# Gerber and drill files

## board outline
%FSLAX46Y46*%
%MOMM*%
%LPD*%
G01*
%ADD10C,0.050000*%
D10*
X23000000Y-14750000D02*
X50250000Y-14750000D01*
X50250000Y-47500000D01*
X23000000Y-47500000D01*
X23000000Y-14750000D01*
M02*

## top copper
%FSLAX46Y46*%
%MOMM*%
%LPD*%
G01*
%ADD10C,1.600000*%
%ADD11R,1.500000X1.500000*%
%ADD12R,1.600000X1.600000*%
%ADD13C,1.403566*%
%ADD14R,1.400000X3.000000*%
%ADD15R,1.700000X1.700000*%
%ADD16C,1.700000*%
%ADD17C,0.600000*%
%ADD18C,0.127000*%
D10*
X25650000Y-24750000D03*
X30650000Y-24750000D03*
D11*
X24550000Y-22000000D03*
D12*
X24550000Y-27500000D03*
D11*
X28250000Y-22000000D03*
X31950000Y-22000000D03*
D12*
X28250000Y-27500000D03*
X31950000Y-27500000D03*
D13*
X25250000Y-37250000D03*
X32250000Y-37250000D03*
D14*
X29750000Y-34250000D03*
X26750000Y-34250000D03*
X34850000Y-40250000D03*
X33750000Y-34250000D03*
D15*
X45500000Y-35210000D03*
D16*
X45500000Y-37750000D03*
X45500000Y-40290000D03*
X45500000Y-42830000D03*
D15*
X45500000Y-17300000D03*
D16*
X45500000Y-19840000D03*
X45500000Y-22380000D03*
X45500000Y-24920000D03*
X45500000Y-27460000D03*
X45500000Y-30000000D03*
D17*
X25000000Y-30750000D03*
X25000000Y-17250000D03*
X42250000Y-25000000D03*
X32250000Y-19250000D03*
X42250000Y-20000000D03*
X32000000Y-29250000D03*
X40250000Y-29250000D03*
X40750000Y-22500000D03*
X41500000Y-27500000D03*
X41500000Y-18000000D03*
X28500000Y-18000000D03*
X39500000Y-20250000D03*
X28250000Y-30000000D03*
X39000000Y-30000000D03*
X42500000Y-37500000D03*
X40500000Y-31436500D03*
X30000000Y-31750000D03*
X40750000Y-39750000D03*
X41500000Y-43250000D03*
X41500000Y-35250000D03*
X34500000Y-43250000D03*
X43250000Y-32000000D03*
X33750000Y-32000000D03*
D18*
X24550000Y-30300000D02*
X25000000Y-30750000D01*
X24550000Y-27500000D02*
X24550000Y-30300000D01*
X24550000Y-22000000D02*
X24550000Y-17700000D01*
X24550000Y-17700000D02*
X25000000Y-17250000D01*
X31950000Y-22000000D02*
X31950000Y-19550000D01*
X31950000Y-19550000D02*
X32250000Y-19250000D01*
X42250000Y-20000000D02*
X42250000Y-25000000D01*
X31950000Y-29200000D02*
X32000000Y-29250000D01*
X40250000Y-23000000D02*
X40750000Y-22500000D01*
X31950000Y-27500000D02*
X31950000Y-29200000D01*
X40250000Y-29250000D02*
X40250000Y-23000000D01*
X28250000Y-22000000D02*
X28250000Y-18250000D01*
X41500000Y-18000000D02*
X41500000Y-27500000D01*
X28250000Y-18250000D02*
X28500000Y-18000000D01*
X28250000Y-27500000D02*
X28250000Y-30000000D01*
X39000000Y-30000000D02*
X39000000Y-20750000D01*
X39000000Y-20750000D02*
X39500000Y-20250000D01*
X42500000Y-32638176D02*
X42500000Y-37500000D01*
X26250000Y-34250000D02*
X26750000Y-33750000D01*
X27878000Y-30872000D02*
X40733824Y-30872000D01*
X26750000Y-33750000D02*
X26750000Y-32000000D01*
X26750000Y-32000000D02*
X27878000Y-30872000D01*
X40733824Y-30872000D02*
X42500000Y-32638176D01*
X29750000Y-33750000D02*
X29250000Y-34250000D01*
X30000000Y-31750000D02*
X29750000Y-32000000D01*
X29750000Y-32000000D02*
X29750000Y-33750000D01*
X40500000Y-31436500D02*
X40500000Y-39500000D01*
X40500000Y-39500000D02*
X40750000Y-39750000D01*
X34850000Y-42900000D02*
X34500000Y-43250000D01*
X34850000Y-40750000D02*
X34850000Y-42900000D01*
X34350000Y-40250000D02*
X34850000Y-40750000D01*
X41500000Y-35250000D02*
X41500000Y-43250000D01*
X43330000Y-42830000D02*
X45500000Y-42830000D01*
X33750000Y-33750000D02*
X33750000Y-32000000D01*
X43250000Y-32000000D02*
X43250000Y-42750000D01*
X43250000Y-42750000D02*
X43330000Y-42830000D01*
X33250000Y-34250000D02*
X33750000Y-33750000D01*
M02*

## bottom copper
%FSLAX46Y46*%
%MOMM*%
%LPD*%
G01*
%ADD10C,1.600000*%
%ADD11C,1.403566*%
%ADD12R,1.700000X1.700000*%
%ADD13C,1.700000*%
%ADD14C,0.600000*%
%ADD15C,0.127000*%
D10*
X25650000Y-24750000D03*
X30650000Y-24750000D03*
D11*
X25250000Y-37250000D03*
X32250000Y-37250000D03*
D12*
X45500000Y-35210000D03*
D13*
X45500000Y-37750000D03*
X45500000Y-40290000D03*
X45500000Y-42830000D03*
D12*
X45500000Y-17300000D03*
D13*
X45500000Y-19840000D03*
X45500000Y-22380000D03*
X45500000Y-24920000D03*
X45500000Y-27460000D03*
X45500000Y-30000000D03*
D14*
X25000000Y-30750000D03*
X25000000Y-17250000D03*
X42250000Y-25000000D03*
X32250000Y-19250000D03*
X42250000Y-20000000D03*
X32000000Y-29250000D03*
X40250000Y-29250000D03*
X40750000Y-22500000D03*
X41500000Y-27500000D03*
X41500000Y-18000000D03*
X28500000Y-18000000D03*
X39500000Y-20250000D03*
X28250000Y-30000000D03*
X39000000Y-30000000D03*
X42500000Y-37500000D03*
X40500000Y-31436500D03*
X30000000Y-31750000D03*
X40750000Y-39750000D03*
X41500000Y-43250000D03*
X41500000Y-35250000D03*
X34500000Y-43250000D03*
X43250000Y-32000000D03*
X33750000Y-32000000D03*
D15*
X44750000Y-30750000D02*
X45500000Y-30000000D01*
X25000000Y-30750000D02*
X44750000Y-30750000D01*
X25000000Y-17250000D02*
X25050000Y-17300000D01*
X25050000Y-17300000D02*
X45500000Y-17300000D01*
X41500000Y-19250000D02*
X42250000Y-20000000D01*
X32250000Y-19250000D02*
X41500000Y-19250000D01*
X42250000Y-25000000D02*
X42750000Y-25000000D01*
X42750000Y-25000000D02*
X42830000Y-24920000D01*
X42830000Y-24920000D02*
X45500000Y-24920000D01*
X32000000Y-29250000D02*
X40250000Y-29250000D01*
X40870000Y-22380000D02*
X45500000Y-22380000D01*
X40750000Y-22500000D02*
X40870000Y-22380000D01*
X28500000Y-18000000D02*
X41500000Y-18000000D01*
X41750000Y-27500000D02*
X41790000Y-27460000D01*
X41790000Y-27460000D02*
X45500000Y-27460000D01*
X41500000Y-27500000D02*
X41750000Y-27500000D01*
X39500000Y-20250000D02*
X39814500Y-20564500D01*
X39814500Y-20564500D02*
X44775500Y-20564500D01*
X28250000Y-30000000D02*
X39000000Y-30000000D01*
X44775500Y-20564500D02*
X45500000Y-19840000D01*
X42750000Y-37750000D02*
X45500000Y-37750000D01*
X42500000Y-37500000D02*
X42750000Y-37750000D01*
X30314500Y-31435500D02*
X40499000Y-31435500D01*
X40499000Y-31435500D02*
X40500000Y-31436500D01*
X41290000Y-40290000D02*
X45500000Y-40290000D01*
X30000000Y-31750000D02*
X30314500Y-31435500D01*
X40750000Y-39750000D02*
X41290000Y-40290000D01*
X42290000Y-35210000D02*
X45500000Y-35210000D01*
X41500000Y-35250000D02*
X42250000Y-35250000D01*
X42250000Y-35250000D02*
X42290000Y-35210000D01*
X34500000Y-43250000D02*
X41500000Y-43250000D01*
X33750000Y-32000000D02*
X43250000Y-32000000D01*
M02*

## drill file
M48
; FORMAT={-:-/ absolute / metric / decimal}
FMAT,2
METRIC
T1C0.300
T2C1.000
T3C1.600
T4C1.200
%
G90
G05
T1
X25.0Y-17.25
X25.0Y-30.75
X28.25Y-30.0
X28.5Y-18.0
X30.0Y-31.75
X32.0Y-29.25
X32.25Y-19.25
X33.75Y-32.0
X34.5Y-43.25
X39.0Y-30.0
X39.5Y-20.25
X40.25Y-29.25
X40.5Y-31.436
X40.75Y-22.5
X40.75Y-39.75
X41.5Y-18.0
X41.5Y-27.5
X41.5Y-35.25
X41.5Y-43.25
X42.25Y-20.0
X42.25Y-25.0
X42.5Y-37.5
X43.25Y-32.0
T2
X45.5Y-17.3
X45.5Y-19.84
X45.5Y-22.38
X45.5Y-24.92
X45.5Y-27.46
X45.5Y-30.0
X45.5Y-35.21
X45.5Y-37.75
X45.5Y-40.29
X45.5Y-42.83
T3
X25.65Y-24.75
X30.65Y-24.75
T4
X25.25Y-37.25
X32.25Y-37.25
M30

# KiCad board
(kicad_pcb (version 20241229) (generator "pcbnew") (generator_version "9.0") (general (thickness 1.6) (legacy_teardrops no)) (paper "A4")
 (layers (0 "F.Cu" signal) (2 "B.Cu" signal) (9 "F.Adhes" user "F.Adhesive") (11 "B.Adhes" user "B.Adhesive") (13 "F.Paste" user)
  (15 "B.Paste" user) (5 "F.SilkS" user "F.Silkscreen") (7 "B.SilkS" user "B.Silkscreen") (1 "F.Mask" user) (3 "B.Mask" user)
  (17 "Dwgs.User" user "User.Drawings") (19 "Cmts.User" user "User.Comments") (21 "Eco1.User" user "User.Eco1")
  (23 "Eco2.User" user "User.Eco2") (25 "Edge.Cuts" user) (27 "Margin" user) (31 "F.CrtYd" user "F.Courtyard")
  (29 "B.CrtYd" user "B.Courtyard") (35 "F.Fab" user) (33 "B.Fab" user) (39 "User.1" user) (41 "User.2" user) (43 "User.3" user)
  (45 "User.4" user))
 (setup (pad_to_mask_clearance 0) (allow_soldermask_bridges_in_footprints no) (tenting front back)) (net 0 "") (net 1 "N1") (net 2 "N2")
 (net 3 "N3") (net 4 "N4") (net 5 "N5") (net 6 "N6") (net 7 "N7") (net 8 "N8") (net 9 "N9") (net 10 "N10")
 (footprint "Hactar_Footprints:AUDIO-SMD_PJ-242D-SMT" (layer "F.Cu") (at 28.25 24.75)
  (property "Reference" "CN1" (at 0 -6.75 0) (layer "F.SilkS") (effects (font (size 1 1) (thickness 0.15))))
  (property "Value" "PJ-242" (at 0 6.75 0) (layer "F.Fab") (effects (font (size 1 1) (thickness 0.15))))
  (pad "" thru_hole circle (at -2.6 0) (size 1.6 1.6) (drill 1.6) (layers "*.Cu" "*.Mask") (remove_unused_layers no))
  (pad "" thru_hole circle (at 2.4 0) (size 1.6 1.6) (drill 1.6) (layers "*.Cu" "*.Mask") (remove_unused_layers no))
  (pad "2" smd rect (at -3.7 -2.75 180) (size 1.5 1.5) (layers "F.Cu" "F.Mask" "F.Paste") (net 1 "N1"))
  (pad "3" smd rect (at -3.7 2.75 180) (size 1.6 1.6) (layers "F.Cu" "F.Mask" "F.Paste") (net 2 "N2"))
  (pad "4" smd rect (at 0 -2.75 180) (size 1.5 1.5) (layers "F.Cu" "F.Mask" "F.Paste") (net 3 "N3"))
  (pad "5" smd rect (at 3.7 -2.75 180) (size 1.5 1.5) (layers "F.Cu" "F.Mask" "F.Paste") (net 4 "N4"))
  (pad "6" smd rect (at 0 2.75 180) (size 1.6 1.6) (layers "F.Cu" "F.Mask" "F.Paste") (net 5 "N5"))
  (pad "7" smd rect (at 3.7 2.75 180) (size 1.6 1.6) (layers "F.Cu" "F.Mask" "F.Paste") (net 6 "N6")))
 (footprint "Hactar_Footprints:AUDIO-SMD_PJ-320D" (layer "F.Cu") (at 30.8 37.25 90)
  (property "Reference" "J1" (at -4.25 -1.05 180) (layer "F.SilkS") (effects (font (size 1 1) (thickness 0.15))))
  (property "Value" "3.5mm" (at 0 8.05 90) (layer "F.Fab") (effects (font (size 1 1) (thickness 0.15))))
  (pad "" np_thru_hole circle (at 0 -5.55 90) (size 1.403566 1.403566) (drill 1.2) (layers "*.Cu" "*.Mask"))
  (pad "" np_thru_hole circle (at 0 1.45 90) (size 1.403566 1.403566) (drill 1.2) (layers "*.Cu" "*.Mask"))
  (pad "R1" smd rect (at 3 -1.05 90) (size 3 1.4) (layers "F.Cu" "F.Mask" "F.Paste") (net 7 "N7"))
  (pad "R2" smd rect (at 3 -4.05 90) (size 3 1.4) (layers "F.Cu" "F.Mask" "F.Paste") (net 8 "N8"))
  (pad "S" smd rect (at -3 4.05 90) (size 3 1.4) (layers "F.Cu" "F.Mask" "F.Paste") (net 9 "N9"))
  (pad "T" smd rect (at 3 2.95 90) (size 3 1.4) (layers "F.Cu" "F.Mask" "F.Paste") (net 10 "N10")))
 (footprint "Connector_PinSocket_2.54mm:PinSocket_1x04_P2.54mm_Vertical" (layer "F.Cu") (at 45.5 35.21)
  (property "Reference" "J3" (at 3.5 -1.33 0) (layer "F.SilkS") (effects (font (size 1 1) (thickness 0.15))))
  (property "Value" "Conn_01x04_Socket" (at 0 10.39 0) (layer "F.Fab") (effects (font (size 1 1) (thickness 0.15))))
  (pad "1" thru_hole rect (at 0 0) (size 1.7 1.7) (drill 1) (layers "*.Cu" "*.Mask") (remove_unused_layers no) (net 9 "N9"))
  (pad "2" thru_hole circle (at 0 2.54) (size 1.7 1.7) (drill 1) (layers "*.Cu" "*.Mask") (remove_unused_layers no) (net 8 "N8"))
  (pad "3" thru_hole circle (at 0 5.08) (size 1.7 1.7) (drill 1) (layers "*.Cu" "*.Mask") (remove_unused_layers no) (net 7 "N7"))
  (pad "4" thru_hole circle (at 0 7.62) (size 1.7 1.7) (drill 1) (layers "*.Cu" "*.Mask") (remove_unused_layers no) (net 10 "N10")))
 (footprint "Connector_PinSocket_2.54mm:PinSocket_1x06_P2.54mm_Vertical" (layer "F.Cu") (at 45.5 17.3)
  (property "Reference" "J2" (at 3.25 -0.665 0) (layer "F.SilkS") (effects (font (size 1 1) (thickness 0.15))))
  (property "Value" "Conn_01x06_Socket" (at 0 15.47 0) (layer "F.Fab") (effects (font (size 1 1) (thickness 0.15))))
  (pad "1" thru_hole rect (at 0 0) (size 1.7 1.7) (drill 1) (layers "*.Cu" "*.Mask") (remove_unused_layers no) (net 1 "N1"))
  (pad "2" thru_hole circle (at 0 2.54) (size 1.7 1.7) (drill 1) (layers "*.Cu" "*.Mask") (remove_unused_layers no) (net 5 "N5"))
  (pad "3" thru_hole circle (at 0 5.08) (size 1.7 1.7) (drill 1) (layers "*.Cu" "*.Mask") (remove_unused_layers no) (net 6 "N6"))
  (pad "4" thru_hole circle (at 0 7.62) (size 1.7 1.7) (drill 1) (layers "*.Cu" "*.Mask") (remove_unused_layers no) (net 4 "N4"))
  (pad "5" thru_hole circle (at 0 10.16) (size 1.7 1.7) (drill 1) (layers "*.Cu" "*.Mask") (remove_unused_layers no) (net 3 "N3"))
  (pad "6" thru_hole circle (at 0 12.7) (size 1.7 1.7) (drill 1) (layers "*.Cu" "*.Mask") (remove_unused_layers no) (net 2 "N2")))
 (gr_rect (start 23 14.75) (end 50.25 47.5) (stroke (width 0.05) (type default)) (fill no) (layer "Edge.Cuts"))
 (segment (start 24.55 30.3) (end 25 30.75) (width 0.127) (layer "F.Cu") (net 2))
 (segment (start 24.55 27.5) (end 24.55 30.3) (width 0.127) (layer "F.Cu") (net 2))
 (via (at 25 30.75) (size 0.6) (drill 0.3) (layers "F.Cu" "B.Cu") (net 2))
 (segment (start 44.75 30.75) (end 45.5 30) (width 0.127) (layer "B.Cu") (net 2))
 (segment (start 25 30.75) (end 44.75 30.75) (width 0.127) (layer "B.Cu") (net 2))
 (segment (start 24.55 22) (end 24.55 17.7) (width 0.127) (layer "F.Cu") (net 1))
 (segment (start 24.55 17.7) (end 25 17.25) (width 0.127) (layer "F.Cu") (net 1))
 (via (at 25 17.25) (size 0.6) (drill 0.3) (layers "F.Cu" "B.Cu") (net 1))
 (segment (start 25 17.25) (end 25.05 17.3) (width 0.127) (layer "B.Cu") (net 1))
 (segment (start 25.05 17.3) (end 45.5 17.3) (width 0.127) (layer "B.Cu") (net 1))
 (segment (start 31.95 22) (end 31.95 19.55) (width 0.127) (layer "F.Cu") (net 4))
 (segment (start 31.95 19.55) (end 32.25 19.25) (width 0.127) (layer "F.Cu") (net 4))
 (segment (start 42.25 20) (end 42.25 25) (width 0.127) (layer "F.Cu") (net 4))
 (via (at 42.25 25) (size 0.6) (drill 0.3) (layers "F.Cu" "B.Cu") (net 4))
 (via (at 32.25 19.25) (size 0.6) (drill 0.3) (layers "F.Cu" "B.Cu") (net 4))
 (via (at 42.25 20) (size 0.6) (drill 0.3) (layers "F.Cu" "B.Cu") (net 4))
 (segment (start 41.5 19.25) (end 42.25 20) (width 0.127) (layer "B.Cu") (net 4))
 (segment (start 32.25 19.25) (end 41.5 19.25) (width 0.127) (layer "B.Cu") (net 4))
 (segment (start 42.25 25) (end 42.75 25) (width 0.127) (layer "B.Cu") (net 4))
 (segment (start 42.75 25) (end 42.83 24.92) (width 0.127) (layer "B.Cu") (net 4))
 (segment (start 42.83 24.92) (end 45.5 24.92) (width 0.127) (layer "B.Cu") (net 4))
 (segment (start 31.95 29.2) (end 32 29.25) (width 0.127) (layer "F.Cu") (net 6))
 (segment (start 40.25 23) (end 40.75 22.5) (width 0.127) (layer "F.Cu") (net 6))
 (segment (start 31.95 27.5) (end 31.95 29.2) (width 0.127) (layer "F.Cu") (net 6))
 (segment (start 40.25 29.25) (end 40.25 23) (width 0.127) (layer "F.Cu") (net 6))
 (via (at 32 29.25) (size 0.6) (drill 0.3) (layers "F.Cu" "B.Cu") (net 6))
 (via (at 40.25 29.25) (size 0.6) (drill 0.3) (layers "F.Cu" "B.Cu") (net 6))
 (via (at 40.75 22.5) (size 0.6) (drill 0.3) (layers "F.Cu" "B.Cu") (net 6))
 (segment (start 32 29.25) (end 40.25 29.25) (width 0.127) (layer "B.Cu") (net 6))
 (segment (start 40.87 22.38) (end 45.5 22.38) (width 0.127) (layer "B.Cu") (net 6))
 (segment (start 40.75 22.5) (end 40.87 22.38) (width 0.127) (layer "B.Cu") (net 6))
 (segment (start 28.25 22) (end 28.25 18.25) (width 0.127) (layer "F.Cu") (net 3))
 (segment (start 41.5 18) (end 41.5 27.5) (width 0.127) (layer "F.Cu") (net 3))
 (segment (start 28.25 18.25) (end 28.5 18) (width 0.127) (layer "F.Cu") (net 3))
 (via (at 41.5 27.5) (size 0.6) (drill 0.3) (layers "F.Cu" "B.Cu") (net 3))
 (via (at 41.5 18) (size 0.6) (drill 0.3) (layers "F.Cu" "B.Cu") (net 3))
 (via (at 28.5 18) (size 0.6) (drill 0.3) (layers "F.Cu" "B.Cu") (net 3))
 (segment (start 28.5 18) (end 41.5 18) (width 0.127) (layer "B.Cu") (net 3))
 (segment (start 41.75 27.5) (end 41.79 27.46) (width 0.127) (layer "B.Cu") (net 3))
 (segment (start 41.79 27.46) (end 45.5 27.46) (width 0.127) (layer "B.Cu") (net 3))
 (segment (start 41.5 27.5) (end 41.75 27.5) (width 0.127) (layer "B.Cu") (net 3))
 (segment (start 28.25 27.5) (end 28.25 30) (width 0.127) (layer "F.Cu") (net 5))
 (segment (start 39 30) (end 39 20.75) (width 0.127) (layer "F.Cu") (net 5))
 (segment (start 39 20.75) (end 39.5 20.25) (width 0.127) (layer "F.Cu") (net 5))
 (via (at 39.5 20.25) (size 0.6) (drill 0.3) (layers "F.Cu" "B.Cu") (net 5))
 (via (at 28.25 30) (size 0.6) (drill 0.3) (layers "F.Cu" "B.Cu") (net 5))
 (via (at 39 30) (size 0.6) (drill 0.3) (layers "F.Cu" "B.Cu") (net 5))
 (segment (start 39.5 20.25) (end 39.8145 20.5645) (width 0.127) (layer "B.Cu") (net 5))
 (segment (start 39.8145 20.5645) (end 44.7755 20.5645) (width 0.127) (layer "B.Cu") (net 5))
 (segment (start 28.25 30) (end 39 30) (width 0.127) (layer "B.Cu") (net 5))
 (segment (start 44.7755 20.5645) (end 45.5 19.84) (width 0.127) (layer "B.Cu") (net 5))
 (segment (start 42.5 32.638176) (end 42.5 37.5) (width 0.127) (layer "F.Cu") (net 8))
 (segment (start 26.25 34.25) (end 26.75 33.75) (width 0.127) (layer "F.Cu") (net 8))
 (segment (start 27.878 30.872) (end 40.733824 30.872) (width 0.127) (layer "F.Cu") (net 8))
 (segment (start 26.75 33.75) (end 26.75 32) (width 0.127) (layer "F.Cu") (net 8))
 (segment (start 26.75 32) (end 27.878 30.872) (width 0.127) (layer "F.Cu") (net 8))
 (segment (start 40.733824 30.872) (end 42.5 32.638176) (width 0.127) (layer "F.Cu") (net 8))
 (via (at 42.5 37.5) (size 0.6) (drill 0.3) (layers "F.Cu" "B.Cu") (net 8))
 (segment (start 42.75 37.75) (end 45.5 37.75) (width 0.127) (layer "B.Cu") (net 8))
 (segment (start 42.5 37.5) (end 42.75 37.75) (width 0.127) (layer "B.Cu") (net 8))
 (segment (start 29.75 33.75) (end 29.25 34.25) (width 0.127) (layer "F.Cu") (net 7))
 (segment (start 30 31.75) (end 29.75 32) (width 0.127) (layer "F.Cu") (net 7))
 (segment (start 29.75 32) (end 29.75 33.75) (width 0.127) (layer "F.Cu") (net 7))
 (segment (start 40.5 31.4365) (end 40.5 39.5) (width 0.127) (layer "F.Cu") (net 7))
 (segment (start 40.5 39.5) (end 40.75 39.75) (width 0.127) (layer "F.Cu") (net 7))
 (via (at 40.5 31.4365) (size 0.6) (drill 0.3) (layers "F.Cu" "B.Cu") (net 7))
 (via (at 30 31.75) (size 0.6) (drill 0.3) (layers "F.Cu" "B.Cu") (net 7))
 (via (at 40.75 39.75) (size 0.6) (drill 0.3) (layers "F.Cu" "B.Cu") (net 7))
 (segment (start 30.3145 31.4355) (end 40.499 31.4355) (width 0.127) (layer "B.Cu") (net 7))
 (segment (start 40.499 31.4355) (end 40.5 31.4365) (width 0.127) (layer "B.Cu") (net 7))
 (segment (start 41.29 40.29) (end 45.5 40.29) (width 0.127) (layer "B.Cu") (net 7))
 (segment (start 30 31.75) (end 30.3145 31.4355) (width 0.127) (layer "B.Cu") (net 7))
 (segment (start 40.75 39.75) (end 41.29 40.29) (width 0.127) (layer "B.Cu") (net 7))
 (segment (start 34.85 42.9) (end 34.5 43.25) (width 0.127) (layer "F.Cu") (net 9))
 (segment (start 34.85 40.75) (end 34.85 42.9) (width 0.127) (layer "F.Cu") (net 9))
 (segment (start 34.35 40.25) (end 34.85 40.75) (width 0.127) (layer "F.Cu") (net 9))
 (segment (start 41.5 35.25) (end 41.5 43.25) (width 0.127) (layer "F.Cu") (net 9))
 (via (at 41.5 43.25) (size 0.6) (drill 0.3) (layers "F.Cu" "B.Cu") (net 9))
 (via (at 41.5 35.25) (size 0.6) (drill 0.3) (layers "F.Cu" "B.Cu") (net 9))
 (via (at 34.5 43.25) (size 0.6) (drill 0.3) (layers "F.Cu" "B.Cu") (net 9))
 (segment (start 42.29 35.21) (end 45.5 35.21) (width 0.127) (layer "B.Cu") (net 9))
 (segment (start 41.5 35.25) (end 42.25 35.25) (width 0.127) (layer "B.Cu") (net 9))
 (segment (start 42.25 35.25) (end 42.29 35.21) (width 0.127) (layer "B.Cu") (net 9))
 (segment (start 34.5 43.25) (end 41.5 43.25) (width 0.127) (layer "B.Cu") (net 9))
 (segment (start 43.33 42.83) (end 45.5 42.83) (width 0.127) (layer "F.Cu") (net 10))
 (segment (start 33.75 33.75) (end 33.75 32) (width 0.127) (layer "F.Cu") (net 10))
 (segment (start 43.25 32) (end 43.25 42.75) (width 0.127) (layer "F.Cu") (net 10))
 (segment (start 43.25 42.75) (end 43.33 42.83) (width 0.127) (layer "F.Cu") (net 10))
 (segment (start 33.25 34.25) (end 33.75 33.75) (width 0.127) (layer "F.Cu") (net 10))
 (via (at 43.25 32) (size 0.6) (drill 0.3) (layers "F.Cu" "B.Cu") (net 10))
 (via (at 33.75 32) (size 0.6) (drill 0.3) (layers "F.Cu" "B.Cu") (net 10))
 (segment (start 33.75 32) (end 43.25 32) (width 0.127) (layer "B.Cu") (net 10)))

